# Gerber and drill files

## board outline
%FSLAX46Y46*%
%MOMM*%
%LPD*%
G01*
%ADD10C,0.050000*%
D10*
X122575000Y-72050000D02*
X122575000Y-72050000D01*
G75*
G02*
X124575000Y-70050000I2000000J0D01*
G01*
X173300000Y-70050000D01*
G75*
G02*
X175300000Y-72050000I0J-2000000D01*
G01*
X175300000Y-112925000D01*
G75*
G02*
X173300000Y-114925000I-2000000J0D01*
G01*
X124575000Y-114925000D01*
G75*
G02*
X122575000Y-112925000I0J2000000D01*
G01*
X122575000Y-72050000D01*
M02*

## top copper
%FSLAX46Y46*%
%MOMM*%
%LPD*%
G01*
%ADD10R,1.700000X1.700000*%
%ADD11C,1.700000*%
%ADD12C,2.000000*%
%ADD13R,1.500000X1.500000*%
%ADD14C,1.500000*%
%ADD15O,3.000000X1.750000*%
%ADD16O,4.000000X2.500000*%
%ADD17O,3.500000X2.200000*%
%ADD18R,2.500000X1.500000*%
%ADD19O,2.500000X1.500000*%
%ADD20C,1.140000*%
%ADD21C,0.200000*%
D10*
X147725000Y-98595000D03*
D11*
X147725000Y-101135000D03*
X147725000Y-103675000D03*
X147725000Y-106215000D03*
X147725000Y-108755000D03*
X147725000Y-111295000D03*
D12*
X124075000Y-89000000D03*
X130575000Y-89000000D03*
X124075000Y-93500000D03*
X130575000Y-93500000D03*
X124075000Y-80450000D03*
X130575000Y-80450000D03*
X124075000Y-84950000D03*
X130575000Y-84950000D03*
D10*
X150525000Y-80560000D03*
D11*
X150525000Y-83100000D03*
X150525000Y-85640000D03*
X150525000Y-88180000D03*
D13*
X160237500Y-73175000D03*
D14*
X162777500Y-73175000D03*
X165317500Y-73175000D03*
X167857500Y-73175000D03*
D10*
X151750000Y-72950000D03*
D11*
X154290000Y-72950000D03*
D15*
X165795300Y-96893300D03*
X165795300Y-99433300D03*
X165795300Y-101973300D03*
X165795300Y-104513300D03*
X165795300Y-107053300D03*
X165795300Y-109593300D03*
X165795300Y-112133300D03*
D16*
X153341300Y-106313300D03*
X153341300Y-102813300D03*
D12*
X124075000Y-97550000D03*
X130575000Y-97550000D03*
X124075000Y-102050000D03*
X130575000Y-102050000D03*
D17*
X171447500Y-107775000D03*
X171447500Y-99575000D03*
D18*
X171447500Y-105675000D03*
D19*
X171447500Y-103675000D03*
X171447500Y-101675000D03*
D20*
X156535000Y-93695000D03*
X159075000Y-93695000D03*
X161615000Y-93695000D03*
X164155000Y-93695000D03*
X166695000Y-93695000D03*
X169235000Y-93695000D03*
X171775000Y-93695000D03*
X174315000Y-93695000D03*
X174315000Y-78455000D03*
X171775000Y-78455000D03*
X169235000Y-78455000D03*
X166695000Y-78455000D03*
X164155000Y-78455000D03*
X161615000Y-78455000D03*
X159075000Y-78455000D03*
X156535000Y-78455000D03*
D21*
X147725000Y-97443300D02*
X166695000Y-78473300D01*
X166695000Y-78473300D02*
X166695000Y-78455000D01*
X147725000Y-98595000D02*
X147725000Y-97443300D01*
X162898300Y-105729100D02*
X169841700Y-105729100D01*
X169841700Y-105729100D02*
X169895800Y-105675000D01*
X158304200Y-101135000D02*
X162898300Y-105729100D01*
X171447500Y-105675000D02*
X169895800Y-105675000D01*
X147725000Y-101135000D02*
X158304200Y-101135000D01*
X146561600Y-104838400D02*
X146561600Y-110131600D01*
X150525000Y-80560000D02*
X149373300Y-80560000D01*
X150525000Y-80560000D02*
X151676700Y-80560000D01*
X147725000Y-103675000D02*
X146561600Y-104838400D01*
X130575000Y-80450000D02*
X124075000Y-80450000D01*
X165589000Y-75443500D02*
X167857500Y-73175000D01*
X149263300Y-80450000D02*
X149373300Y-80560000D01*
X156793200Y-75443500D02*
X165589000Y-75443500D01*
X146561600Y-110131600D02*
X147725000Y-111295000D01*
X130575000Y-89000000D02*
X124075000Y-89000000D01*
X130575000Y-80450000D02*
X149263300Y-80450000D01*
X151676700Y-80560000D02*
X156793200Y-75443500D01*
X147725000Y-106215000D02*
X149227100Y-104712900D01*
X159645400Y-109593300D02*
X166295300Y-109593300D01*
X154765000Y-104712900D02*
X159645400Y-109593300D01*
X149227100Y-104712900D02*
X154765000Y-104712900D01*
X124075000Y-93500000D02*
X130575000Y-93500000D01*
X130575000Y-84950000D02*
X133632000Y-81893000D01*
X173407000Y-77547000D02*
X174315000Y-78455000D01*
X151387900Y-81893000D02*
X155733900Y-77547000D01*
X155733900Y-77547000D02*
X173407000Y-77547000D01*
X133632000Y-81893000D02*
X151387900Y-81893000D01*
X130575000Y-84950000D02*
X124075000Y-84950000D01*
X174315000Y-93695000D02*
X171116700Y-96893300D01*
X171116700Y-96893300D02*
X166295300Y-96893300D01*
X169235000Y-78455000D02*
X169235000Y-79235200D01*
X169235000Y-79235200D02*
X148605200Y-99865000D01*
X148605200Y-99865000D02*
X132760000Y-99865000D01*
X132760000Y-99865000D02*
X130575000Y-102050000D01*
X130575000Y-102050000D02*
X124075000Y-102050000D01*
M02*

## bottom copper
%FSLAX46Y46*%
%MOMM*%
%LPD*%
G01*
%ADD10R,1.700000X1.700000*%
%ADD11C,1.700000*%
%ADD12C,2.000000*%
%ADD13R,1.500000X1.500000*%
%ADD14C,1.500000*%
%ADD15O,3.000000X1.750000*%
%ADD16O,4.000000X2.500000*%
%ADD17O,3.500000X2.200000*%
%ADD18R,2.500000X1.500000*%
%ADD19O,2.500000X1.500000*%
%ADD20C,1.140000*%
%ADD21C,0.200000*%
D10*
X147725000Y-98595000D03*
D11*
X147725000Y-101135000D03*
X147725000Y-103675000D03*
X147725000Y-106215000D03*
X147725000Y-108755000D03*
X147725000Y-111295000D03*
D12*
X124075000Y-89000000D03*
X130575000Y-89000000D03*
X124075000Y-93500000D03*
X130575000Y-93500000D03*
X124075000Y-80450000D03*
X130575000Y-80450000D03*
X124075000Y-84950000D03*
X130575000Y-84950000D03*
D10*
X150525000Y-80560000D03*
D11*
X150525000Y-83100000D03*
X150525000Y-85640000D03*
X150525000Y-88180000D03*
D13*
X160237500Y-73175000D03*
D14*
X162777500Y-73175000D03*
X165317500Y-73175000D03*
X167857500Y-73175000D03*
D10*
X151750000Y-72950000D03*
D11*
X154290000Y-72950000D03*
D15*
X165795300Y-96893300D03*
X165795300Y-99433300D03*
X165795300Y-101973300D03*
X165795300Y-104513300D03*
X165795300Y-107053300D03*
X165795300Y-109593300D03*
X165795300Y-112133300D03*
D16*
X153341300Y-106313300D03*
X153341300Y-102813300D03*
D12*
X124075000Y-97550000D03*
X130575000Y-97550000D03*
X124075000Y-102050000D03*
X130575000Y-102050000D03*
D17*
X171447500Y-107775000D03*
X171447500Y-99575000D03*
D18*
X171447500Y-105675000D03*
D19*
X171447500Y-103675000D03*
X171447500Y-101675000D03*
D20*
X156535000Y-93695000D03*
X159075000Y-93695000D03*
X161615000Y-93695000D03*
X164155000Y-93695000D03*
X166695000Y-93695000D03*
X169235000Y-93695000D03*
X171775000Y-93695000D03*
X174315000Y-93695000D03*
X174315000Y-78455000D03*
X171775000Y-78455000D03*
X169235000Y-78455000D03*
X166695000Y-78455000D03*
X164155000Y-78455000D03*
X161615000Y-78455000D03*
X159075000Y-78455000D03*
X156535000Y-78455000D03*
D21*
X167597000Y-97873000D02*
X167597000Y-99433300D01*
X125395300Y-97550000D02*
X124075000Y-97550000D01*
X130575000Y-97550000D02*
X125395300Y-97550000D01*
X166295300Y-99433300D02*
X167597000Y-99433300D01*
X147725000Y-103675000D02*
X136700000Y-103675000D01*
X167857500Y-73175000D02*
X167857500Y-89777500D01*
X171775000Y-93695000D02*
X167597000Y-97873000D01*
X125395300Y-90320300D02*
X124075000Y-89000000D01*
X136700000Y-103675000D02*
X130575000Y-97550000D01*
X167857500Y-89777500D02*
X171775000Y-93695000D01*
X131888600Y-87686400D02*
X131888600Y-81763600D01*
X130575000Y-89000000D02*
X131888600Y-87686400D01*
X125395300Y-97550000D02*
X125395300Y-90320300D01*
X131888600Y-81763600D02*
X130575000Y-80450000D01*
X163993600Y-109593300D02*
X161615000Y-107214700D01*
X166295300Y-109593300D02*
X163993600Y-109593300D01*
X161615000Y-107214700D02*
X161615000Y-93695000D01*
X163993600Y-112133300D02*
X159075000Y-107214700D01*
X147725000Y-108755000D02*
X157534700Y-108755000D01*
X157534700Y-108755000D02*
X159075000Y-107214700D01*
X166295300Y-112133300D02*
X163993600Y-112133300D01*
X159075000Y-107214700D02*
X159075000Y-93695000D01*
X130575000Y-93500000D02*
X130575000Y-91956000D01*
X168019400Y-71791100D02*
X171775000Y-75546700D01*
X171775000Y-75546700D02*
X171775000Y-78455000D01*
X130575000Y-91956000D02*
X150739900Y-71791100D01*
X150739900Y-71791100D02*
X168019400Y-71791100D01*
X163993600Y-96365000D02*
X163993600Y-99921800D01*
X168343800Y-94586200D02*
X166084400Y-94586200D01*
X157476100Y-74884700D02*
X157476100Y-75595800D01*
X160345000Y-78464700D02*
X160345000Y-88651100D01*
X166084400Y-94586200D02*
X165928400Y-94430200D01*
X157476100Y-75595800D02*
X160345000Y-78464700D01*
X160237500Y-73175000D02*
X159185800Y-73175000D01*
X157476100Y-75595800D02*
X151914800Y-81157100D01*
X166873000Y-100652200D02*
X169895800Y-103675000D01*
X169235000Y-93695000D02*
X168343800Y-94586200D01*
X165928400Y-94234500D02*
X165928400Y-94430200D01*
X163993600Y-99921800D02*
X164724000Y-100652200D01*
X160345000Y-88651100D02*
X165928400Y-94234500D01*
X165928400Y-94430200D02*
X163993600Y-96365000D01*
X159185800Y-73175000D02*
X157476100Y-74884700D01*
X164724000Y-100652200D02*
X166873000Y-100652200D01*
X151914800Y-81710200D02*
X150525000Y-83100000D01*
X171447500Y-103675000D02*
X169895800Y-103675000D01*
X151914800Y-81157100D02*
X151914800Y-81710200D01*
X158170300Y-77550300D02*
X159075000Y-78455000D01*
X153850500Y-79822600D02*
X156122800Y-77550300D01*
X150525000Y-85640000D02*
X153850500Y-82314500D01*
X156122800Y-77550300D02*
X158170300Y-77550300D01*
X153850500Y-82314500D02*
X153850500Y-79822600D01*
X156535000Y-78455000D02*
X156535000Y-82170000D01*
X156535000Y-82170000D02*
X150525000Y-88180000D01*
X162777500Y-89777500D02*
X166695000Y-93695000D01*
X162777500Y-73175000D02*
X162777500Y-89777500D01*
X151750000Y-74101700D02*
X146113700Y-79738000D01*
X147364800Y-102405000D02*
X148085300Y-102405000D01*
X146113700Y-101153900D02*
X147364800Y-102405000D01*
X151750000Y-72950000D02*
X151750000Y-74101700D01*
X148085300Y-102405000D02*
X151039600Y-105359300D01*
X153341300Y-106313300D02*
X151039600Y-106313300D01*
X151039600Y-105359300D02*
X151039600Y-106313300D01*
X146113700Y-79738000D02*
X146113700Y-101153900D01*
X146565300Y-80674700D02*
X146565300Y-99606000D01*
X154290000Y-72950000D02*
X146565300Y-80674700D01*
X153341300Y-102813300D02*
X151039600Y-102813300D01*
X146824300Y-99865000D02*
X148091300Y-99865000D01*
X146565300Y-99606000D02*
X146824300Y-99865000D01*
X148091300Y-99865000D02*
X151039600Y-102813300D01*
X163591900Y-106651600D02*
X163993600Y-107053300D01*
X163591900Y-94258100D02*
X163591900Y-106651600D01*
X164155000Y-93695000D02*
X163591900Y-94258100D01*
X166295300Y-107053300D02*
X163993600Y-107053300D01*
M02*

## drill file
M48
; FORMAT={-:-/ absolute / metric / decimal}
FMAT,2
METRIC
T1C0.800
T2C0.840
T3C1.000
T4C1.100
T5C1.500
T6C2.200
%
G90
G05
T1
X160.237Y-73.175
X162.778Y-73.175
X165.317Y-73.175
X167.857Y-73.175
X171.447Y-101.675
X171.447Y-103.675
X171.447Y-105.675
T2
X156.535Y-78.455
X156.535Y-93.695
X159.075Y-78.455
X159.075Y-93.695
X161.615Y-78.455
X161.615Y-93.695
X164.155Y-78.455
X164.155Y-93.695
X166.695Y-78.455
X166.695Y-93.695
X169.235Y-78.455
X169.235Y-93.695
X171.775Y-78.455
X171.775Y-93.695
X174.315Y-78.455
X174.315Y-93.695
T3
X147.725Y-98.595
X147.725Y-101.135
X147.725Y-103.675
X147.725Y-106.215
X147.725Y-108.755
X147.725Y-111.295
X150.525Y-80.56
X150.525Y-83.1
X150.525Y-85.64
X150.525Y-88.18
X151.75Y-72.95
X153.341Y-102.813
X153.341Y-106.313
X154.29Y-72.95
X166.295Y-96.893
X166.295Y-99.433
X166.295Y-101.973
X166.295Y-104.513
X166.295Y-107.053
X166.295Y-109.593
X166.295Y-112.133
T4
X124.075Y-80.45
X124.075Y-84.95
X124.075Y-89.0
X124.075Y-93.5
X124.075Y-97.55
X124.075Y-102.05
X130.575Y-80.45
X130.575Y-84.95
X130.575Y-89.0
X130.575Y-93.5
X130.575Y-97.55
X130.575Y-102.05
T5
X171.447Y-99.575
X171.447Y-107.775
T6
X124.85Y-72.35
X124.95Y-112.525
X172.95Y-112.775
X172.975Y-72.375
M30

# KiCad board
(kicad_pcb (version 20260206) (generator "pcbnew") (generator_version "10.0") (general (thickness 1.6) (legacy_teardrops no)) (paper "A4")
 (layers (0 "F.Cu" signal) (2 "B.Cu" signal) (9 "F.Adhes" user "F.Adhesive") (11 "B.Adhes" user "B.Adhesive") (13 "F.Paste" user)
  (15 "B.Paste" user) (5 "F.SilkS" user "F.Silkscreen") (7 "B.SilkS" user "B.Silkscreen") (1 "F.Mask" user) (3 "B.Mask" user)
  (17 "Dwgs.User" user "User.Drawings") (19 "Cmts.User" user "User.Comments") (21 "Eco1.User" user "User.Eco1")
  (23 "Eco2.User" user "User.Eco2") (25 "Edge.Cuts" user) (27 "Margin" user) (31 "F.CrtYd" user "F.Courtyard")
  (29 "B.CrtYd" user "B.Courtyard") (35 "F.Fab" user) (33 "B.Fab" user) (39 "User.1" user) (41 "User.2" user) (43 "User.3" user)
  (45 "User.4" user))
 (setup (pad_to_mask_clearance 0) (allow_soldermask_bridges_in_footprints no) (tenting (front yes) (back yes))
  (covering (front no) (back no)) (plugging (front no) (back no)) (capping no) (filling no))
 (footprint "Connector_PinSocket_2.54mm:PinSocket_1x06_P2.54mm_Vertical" (layer "F.Cu") (at 147.725 98.595)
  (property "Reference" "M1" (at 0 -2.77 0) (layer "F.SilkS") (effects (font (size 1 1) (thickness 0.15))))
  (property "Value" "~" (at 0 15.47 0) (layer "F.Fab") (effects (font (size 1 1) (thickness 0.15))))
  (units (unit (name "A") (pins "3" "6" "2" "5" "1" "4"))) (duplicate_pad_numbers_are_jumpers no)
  (pad "1" thru_hole rect (at 0 0) (size 1.7 1.7) (drill 1) (layers "*.Cu" "*.Mask") (remove_unused_layers no) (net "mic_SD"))
  (pad "2" thru_hole circle (at 0 2.54) (size 1.7 1.7) (drill 1) (layers "*.Cu" "*.Mask") (remove_unused_layers no) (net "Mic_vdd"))
  (pad "3" thru_hole circle (at 0 5.08) (size 1.7 1.7) (drill 1) (layers "*.Cu" "*.Mask") (remove_unused_layers no) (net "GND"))
  (pad "4" thru_hole circle (at 0 7.62) (size 1.7 1.7) (drill 1) (layers "*.Cu" "*.Mask") (remove_unused_layers no) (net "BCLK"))
  (pad "5" thru_hole circle (at 0 10.16) (size 1.7 1.7) (drill 1) (layers "*.Cu" "*.Mask") (remove_unused_layers no) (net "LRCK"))
  (pad "6" thru_hole circle (at 0 12.7) (size 1.7 1.7) (drill 1) (layers "*.Cu" "*.Mask") (remove_unused_layers no) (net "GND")))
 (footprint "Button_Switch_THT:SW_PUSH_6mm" (layer "F.Cu") (at 124.075 89)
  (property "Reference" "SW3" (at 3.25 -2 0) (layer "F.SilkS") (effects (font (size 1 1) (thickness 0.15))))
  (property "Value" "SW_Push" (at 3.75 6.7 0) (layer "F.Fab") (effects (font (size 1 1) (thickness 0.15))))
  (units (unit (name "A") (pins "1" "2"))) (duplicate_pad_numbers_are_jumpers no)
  (pad "1" thru_hole circle (at 0 0 90) (size 2 2) (drill 1.1) (layers "*.Cu" "*.Mask") (remove_unused_layers no) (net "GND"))
  (pad "1" thru_hole circle (at 6.5 0 90) (size 2 2) (drill 1.1) (layers "*.Cu" "*.Mask") (remove_unused_layers no) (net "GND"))
  (pad "2" thru_hole circle (at 0 4.5 90) (size 2 2) (drill 1.1) (layers "*.Cu" "*.Mask") (remove_unused_layers no) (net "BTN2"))
  (pad "2" thru_hole circle (at 6.5 4.5 90) (size 2 2) (drill 1.1) (layers "*.Cu" "*.Mask") (remove_unused_layers no) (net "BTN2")))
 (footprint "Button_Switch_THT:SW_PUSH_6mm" (layer "F.Cu") (at 124.075 80.45)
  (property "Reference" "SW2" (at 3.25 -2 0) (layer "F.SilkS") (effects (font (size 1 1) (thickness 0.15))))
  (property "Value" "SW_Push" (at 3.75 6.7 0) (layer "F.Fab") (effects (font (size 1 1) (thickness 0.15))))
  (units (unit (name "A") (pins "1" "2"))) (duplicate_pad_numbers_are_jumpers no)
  (pad "1" thru_hole circle (at 0 0 90) (size 2 2) (drill 1.1) (layers "*.Cu" "*.Mask") (remove_unused_layers no) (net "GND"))
  (pad "1" thru_hole circle (at 6.5 0 90) (size 2 2) (drill 1.1) (layers "*.Cu" "*.Mask") (remove_unused_layers no) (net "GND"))
  (pad "2" thru_hole circle (at 0 4.5 90) (size 2 2) (drill 1.1) (layers "*.Cu" "*.Mask") (remove_unused_layers no) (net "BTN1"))
  (pad "2" thru_hole circle (at 6.5 4.5 90) (size 2 2) (drill 1.1) (layers "*.Cu" "*.Mask") (remove_unused_layers no) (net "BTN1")))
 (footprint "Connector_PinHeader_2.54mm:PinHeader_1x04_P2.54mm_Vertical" (layer "F.Cu") (at 150.525 80.56)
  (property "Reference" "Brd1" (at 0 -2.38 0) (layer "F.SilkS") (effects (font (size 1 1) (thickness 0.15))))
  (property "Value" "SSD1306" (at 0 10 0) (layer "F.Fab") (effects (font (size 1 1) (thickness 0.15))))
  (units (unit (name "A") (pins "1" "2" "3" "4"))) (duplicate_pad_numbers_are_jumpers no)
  (pad "1" thru_hole rect (at 0 0) (size 1.7 1.7) (drill 1) (layers "*.Cu" "*.Mask") (remove_unused_layers no) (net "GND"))
  (pad "2" thru_hole circle (at 0 2.54) (size 1.7 1.7) (drill 1) (layers "*.Cu" "*.Mask") (remove_unused_layers no) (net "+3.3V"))
  (pad "3" thru_hole circle (at 0 5.08) (size 1.7 1.7) (drill 1) (layers "*.Cu" "*.Mask") (remove_unused_layers no) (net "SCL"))
  (pad "4" thru_hole circle (at 0 7.62) (size 1.7 1.7) (drill 1) (layers "*.Cu" "*.Mask") (remove_unused_layers no) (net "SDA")))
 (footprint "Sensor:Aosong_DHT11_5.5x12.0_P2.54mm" (layer "F.Cu") (at 160.2375 73.175 90)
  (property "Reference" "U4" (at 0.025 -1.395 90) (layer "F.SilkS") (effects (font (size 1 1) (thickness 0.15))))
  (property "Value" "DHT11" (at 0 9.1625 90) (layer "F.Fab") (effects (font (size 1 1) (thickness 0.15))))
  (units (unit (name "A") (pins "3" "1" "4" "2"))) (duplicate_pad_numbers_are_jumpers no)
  (pad "1" thru_hole rect (at 0 0 90) (size 1.5 1.5) (drill 0.8) (layers "*.Cu" "*.Mask") (remove_unused_layers no) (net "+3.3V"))
  (pad "2" thru_hole circle (at 0 2.54 90) (size 1.5 1.5) (drill 0.8) (layers "*.Cu" "*.Mask") (remove_unused_layers no) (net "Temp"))
  (pad "3" thru_hole circle (at 0 5.08 90) (size 1.5 1.5) (drill 0.8) (layers "*.Cu" "*.Mask") (remove_unused_layers no)
   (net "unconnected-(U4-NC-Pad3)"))
  (pad "4" thru_hole circle (at 0 7.62 90) (size 1.5 1.5) (drill 0.8) (layers "*.Cu" "*.Mask") (remove_unused_layers no) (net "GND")))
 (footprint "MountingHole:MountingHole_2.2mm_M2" (layer "F.Cu") (at 172.975 72.375)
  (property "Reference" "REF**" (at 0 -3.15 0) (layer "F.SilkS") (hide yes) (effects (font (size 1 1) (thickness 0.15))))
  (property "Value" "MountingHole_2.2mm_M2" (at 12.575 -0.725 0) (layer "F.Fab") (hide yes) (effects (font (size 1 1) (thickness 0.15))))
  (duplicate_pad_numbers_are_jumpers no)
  (pad "" np_thru_hole circle (at 0 0) (size 2.2 2.2) (drill 2.2) (layers "*.Cu" "*.Mask")))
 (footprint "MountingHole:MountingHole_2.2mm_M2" (layer "F.Cu") (at 124.95 112.525)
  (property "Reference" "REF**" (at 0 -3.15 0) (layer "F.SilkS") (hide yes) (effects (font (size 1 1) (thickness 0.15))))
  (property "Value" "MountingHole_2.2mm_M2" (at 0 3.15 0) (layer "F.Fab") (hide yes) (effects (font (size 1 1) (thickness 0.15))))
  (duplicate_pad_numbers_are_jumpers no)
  (pad "" np_thru_hole circle (at 0 0) (size 2.2 2.2) (drill 2.2) (layers "*.Cu" "*.Mask")))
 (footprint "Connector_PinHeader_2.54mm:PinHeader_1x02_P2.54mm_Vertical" (layer "F.Cu") (at 151.75 72.95 90)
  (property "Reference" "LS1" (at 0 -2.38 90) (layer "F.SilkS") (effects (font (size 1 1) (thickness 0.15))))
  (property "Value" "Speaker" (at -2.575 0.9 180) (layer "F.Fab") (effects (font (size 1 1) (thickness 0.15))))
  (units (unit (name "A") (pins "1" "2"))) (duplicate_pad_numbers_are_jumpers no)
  (pad "1" thru_hole rect (at 0 0 90) (size 1.7 1.7) (drill 1) (layers "*.Cu" "*.Mask") (remove_unused_layers no) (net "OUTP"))
  (pad "2" thru_hole circle (at 0 2.54 90) (size 1.7 1.7) (drill 1) (layers "*.Cu" "*.Mask") (remove_unused_layers no) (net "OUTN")))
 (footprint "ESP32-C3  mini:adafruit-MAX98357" (layer "F.Cu") (at 159.3883 104.3933 90)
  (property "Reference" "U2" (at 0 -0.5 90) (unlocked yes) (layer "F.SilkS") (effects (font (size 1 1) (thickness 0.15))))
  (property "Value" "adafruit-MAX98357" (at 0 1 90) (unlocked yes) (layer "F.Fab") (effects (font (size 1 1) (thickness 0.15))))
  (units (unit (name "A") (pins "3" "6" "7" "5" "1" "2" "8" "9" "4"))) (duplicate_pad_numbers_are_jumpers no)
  (pad "1" thru_hole oval (at 7.5 6.907) (size 3 1.75) (drill 1 (offset -0.5 0)) (layers "*.Cu" "*.Mask") (remove_unused_layers no)
   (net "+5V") (solder_mask_margin 0.0508))
  (pad "2" thru_hole oval (at 4.96 6.907) (size 3 1.75) (drill 1 (offset -0.5 0)) (layers "*.Cu" "*.Mask") (remove_unused_layers no)
   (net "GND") (solder_mask_margin 0.0508))
  (pad "3" thru_hole oval (at 2.42 6.907) (size 3 1.75) (drill 1 (offset -0.5 0)) (layers "*.Cu" "*.Mask") (remove_unused_layers no)
   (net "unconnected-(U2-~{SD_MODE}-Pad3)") (solder_mask_margin 0.0508))
  (pad "4" thru_hole oval (at -0.12 6.907) (size 3 1.75) (drill 1 (offset -0.5 0)) (layers "*.Cu" "*.Mask") (remove_unused_layers no)
   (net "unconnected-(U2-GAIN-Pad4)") (solder_mask_margin 0.0508))
  (pad "5" thru_hole oval (at -2.66 6.907) (size 3 1.75) (drill 1 (offset -0.5 0)) (layers "*.Cu" "*.Mask") (remove_unused_layers no)
   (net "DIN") (solder_mask_margin 0.0508))
  (pad "6" thru_hole oval (at -5.2 6.907) (size 3 1.75) (drill 1 (offset -0.5 0)) (layers "*.Cu" "*.Mask") (remove_unused_layers no)
   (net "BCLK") (solder_mask_margin 0.0508))
  (pad "7" thru_hole oval (at -7.74 6.907) (size 3 1.75) (drill 1 (offset -0.5 0)) (layers "*.Cu" "*.Mask") (remove_unused_layers no)
   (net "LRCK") (solder_mask_margin 0.0508))
  (pad "8" thru_hole oval (at -1.92 -6.047 270) (size 2.5 4) (drill 1) (layers "*.Cu" "*.Mask") (remove_unused_layers no) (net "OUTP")
   (solder_mask_margin 0.0508))
  (pad "9" thru_hole oval (at 1.58 -6.047 270) (size 2.5 4) (drill 1) (layers "*.Cu" "*.Mask") (remove_unused_layers no) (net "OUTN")
   (solder_mask_margin 0.0508)))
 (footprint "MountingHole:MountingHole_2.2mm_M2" (layer "F.Cu") (at 172.95 112.775)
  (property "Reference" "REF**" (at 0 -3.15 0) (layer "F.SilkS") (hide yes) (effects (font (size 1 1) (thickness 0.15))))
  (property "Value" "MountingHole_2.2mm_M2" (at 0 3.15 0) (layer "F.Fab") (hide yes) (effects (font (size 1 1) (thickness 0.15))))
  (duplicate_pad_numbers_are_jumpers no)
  (pad "" np_thru_hole circle (at 0 0) (size 2.2 2.2) (drill 2.2) (layers "*.Cu" "*.Mask")))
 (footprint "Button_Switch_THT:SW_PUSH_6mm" (layer "F.Cu") (at 124.075 97.55)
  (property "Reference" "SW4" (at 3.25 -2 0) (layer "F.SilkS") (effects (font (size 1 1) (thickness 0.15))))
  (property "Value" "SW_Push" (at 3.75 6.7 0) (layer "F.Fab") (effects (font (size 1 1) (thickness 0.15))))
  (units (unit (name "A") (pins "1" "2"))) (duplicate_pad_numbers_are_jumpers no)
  (pad "1" thru_hole circle (at 0 0 90) (size 2 2) (drill 1.1) (layers "*.Cu" "*.Mask") (remove_unused_layers no) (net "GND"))
  (pad "1" thru_hole circle (at 6.5 0 90) (size 2 2) (drill 1.1) (layers "*.Cu" "*.Mask") (remove_unused_layers no) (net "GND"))
  (pad "2" thru_hole circle (at 0 4.5 90) (size 2 2) (drill 1.1) (layers "*.Cu" "*.Mask") (remove_unused_layers no) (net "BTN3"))
  (pad "2" thru_hole circle (at 6.5 4.5 90) (size 2 2) (drill 1.1) (layers "*.Cu" "*.Mask") (remove_unused_layers no) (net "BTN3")))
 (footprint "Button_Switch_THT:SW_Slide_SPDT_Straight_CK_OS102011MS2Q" (layer "F.Cu") (at 171.4475 105.675 90)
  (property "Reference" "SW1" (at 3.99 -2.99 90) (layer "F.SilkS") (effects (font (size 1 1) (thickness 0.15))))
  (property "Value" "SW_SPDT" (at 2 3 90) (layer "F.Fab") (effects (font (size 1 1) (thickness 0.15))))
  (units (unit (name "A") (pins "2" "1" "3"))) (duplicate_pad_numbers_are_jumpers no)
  (pad "" thru_hole oval (at -2.1 0 90) (size 2.2 3.5) (drill 1.5) (layers "*.Cu" "*.Mask") (remove_unused_layers no))
  (pad "" thru_hole oval (at 6.1 0 90) (size 2.2 3.5) (drill 1.5) (layers "*.Cu" "*.Mask") (remove_unused_layers no))
  (pad "1" thru_hole rect (at 0 0 90) (size 1.5 2.5) (drill 0.8) (layers "*.Cu" "*.Mask") (remove_unused_layers no) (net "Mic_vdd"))
  (pad "2" thru_hole oval (at 2 0 90) (size 1.5 2.5) (drill 0.8) (layers "*.Cu" "*.Mask") (remove_unused_layers no) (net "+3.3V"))
  (pad "3" thru_hole oval (at 4 0 90) (size 1.5 2.5) (drill 0.8) (layers "*.Cu" "*.Mask") (remove_unused_layers no)
   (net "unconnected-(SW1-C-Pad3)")))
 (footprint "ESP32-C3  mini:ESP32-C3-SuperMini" (layer "F.Cu") (at 165.425 86.075 -90)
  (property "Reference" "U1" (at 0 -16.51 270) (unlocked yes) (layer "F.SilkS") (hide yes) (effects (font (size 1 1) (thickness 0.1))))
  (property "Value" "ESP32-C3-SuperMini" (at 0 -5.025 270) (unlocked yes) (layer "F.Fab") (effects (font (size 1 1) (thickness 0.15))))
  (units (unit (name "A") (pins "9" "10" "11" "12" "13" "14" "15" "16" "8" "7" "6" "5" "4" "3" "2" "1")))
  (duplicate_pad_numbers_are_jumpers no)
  (pad "1" thru_hole circle (at 7.62 8.89 270) (size 1.14 1.14) (drill 0.84) (layers "*.Cu" "*.Mask") (remove_unused_layers no)
   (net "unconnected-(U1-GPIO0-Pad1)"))
  (pad "2" thru_hole circle (at 7.62 6.35 270) (size 1.14 1.14) (drill 0.84) (layers "*.Cu" "*.Mask") (remove_unused_layers no) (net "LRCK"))
  (pad "3" thru_hole circle (at 7.62 3.81 270) (size 1.14 1.14) (drill 0.84) (layers "*.Cu" "*.Mask") (remove_unused_layers no) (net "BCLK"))
  (pad "4" thru_hole circle (at 7.62 1.27 270) (size 1.14 1.14) (drill 0.84) (layers "*.Cu" "*.Mask") (remove_unused_layers no) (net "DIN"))
  (pad "5" thru_hole circle (at 7.62 -1.27 270) (size 1.14 1.14) (drill 0.84) (layers "*.Cu" "*.Mask") (remove_unused_layers no)
   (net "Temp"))
  (pad "6" thru_hole circle (at 7.62 -3.81 270) (size 1.14 1.14) (drill 0.84) (layers "*.Cu" "*.Mask") (remove_unused_layers no)
   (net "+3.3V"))
  (pad "7" thru_hole circle (at 7.62 -6.35 270) (size 1.14 1.14) (drill 0.84) (layers "*.Cu" "*.Mask") (remove_unused_layers no) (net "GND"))
  (pad "8" thru_hole circle (at 7.62 -8.89 270) (size 1.14 1.14) (drill 0.84) (layers "*.Cu" "*.Mask") (remove_unused_layers no) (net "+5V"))
  (pad "9" thru_hole circle (at -7.62 -8.89 270) (size 1.14 1.14) (drill 0.84) (layers "*.Cu" "*.Mask") (remove_unused_layers no)
   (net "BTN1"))
  (pad "10" thru_hole circle (at -7.62 -6.35 270) (size 1.14 1.14) (drill 0.84) (layers "*.Cu" "*.Mask") (remove_unused_layers no)
   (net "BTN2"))
  (pad "11" thru_hole circle (at -7.62 -3.81 270) (size 1.14 1.14) (drill 0.84) (layers "*.Cu" "*.Mask") (remove_unused_layers no)
   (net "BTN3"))
  (pad "12" thru_hole circle (at -7.62 -1.27 270) (size 1.14 1.14) (drill 0.84) (layers "*.Cu" "*.Mask") (remove_unused_layers no)
   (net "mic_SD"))
  (pad "13" thru_hole circle (at -7.62 1.27 270) (size 1.14 1.14) (drill 0.84) (layers "*.Cu" "*.Mask") (remove_unused_layers no)
   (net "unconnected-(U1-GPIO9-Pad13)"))
  (pad "14" thru_hole circle (at -7.62 3.81 270) (size 1.14 1.14) (drill 0.84) (layers "*.Cu" "*.Mask") (remove_unused_layers no)
   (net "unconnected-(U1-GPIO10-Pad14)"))
  (pad "15" thru_hole circle (at -7.62 6.35 270) (size 1.14 1.14) (drill 0.84) (layers "*.Cu" "*.Mask") (remove_unused_layers no)
   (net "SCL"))
  (pad "16" thru_hole circle (at -7.62 8.89 270) (size 1.14 1.14) (drill 0.84) (layers "*.Cu" "*.Mask") (remove_unused_layers no)
   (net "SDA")))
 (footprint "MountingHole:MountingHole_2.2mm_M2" (layer "F.Cu") (at 124.85 72.35)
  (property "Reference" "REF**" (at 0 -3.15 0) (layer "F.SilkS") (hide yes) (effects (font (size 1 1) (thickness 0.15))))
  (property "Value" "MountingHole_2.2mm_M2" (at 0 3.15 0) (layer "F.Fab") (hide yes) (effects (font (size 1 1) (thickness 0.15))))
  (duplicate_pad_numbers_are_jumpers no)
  (pad "" np_thru_hole circle (at 0 0) (size 2.2 2.2) (drill 2.2) (layers "*.Cu" "*.Mask")))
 (gr_rect (start 122.575 70.05) (end 175.3 114.925) (radius 2) (stroke (width 0.05) (type solid)) (fill no) (layer "Edge.Cuts"))
 (segment (start 147.725 97.4433) (end 166.695 78.4733) (width 0.2) (layer "F.Cu") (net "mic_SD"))
 (segment (start 166.695 78.4733) (end 166.695 78.455) (width 0.2) (layer "F.Cu") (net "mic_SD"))
 (segment (start 147.725 98.595) (end 147.725 97.4433) (width 0.2) (layer "F.Cu") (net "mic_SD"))
 (segment (start 162.8983 105.7291) (end 169.8417 105.7291) (width 0.2) (layer "F.Cu") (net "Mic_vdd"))
 (segment (start 169.8417 105.7291) (end 169.8958 105.675) (width 0.2) (layer "F.Cu") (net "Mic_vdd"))
 (segment (start 158.3042 101.135) (end 162.8983 105.7291) (width 0.2) (layer "F.Cu") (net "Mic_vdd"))
 (segment (start 171.4475 105.675) (end 169.8958 105.675) (width 0.2) (layer "F.Cu") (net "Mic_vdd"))
 (segment (start 147.725 101.135) (end 158.3042 101.135) (width 0.2) (layer "F.Cu") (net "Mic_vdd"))
 (segment (start 146.5616 104.8384) (end 146.5616 110.1316) (width 0.2) (layer "F.Cu") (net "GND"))
 (segment (start 150.525 80.56) (end 149.3733 80.56) (width 0.2) (layer "F.Cu") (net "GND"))
 (segment (start 150.525 80.56) (end 151.6767 80.56) (width 0.2) (layer "F.Cu") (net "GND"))
 (segment (start 147.725 103.675) (end 146.5616 104.8384) (width 0.2) (layer "F.Cu") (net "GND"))
 (segment (start 130.575 80.45) (end 124.075 80.45) (width 0.2) (layer "F.Cu") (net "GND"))
 (segment (start 165.589 75.4435) (end 167.8575 73.175) (width 0.2) (layer "F.Cu") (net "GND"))
 (segment (start 149.2633 80.45) (end 149.3733 80.56) (width 0.2) (layer "F.Cu") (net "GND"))
 (segment (start 156.7932 75.4435) (end 165.589 75.4435) (width 0.2) (layer "F.Cu") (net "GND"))
 (segment (start 146.5616 110.1316) (end 147.725 111.295) (width 0.2) (layer "F.Cu") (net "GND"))
 (segment (start 130.575 89) (end 124.075 89) (width 0.2) (layer "F.Cu") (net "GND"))
 (segment (start 130.575 80.45) (end 149.2633 80.45) (width 0.2) (layer "F.Cu") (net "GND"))
 (segment (start 151.6767 80.56) (end 156.7932 75.4435) (width 0.2) (layer "F.Cu") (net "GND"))
 (segment (start 167.597 97.873) (end 167.597 99.4333) (width 0.2) (layer "B.Cu") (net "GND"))
 (segment (start 125.3953 97.55) (end 124.075 97.55) (width 0.2) (layer "B.Cu") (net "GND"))
 (segment (start 130.575 97.55) (end 125.3953 97.55) (width 0.2) (layer "B.Cu") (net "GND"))
 (segment (start 166.2953 99.4333) (end 167.597 99.4333) (width 0.2) (layer "B.Cu") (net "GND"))
 (segment (start 147.725 103.675) (end 136.7 103.675) (width 0.2) (layer "B.Cu") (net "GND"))
 (segment (start 167.8575 73.175) (end 167.8575 89.7775) (width 0.2) (layer "B.Cu") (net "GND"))
 (segment (start 171.775 93.695) (end 167.597 97.873) (width 0.2) (layer "B.Cu") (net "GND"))
 (segment (start 125.3953 90.3203) (end 124.075 89) (width 0.2) (layer "B.Cu") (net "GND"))
 (segment (start 136.7 103.675) (end 130.575 97.55) (width 0.2) (layer "B.Cu") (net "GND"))
 (segment (start 167.8575 89.7775) (end 171.775 93.695) (width 0.2) (layer "B.Cu") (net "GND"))
 (segment (start 131.8886 87.6864) (end 131.8886 81.7636) (width 0.2) (layer "B.Cu") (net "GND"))
 (segment (start 130.575 89) (end 131.8886 87.6864) (width 0.2) (layer "B.Cu") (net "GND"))
 (segment (start 125.3953 97.55) (end 125.3953 90.3203) (width 0.2) (layer "B.Cu") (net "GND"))
 (segment (start 131.8886 81.7636) (end 130.575 80.45) (width 0.2) (layer "B.Cu") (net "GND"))
 (segment (start 147.725 106.215) (end 149.2271 104.7129) (width 0.2) (layer "F.Cu") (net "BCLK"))
 (segment (start 159.6454 109.5933) (end 166.2953 109.5933) (width 0.2) (layer "F.Cu") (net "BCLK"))
 (segment (start 154.765 104.7129) (end 159.6454 109.5933) (width 0.2) (layer "F.Cu") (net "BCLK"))
 (segment (start 149.2271 104.7129) (end 154.765 104.7129) (width 0.2) (layer "F.Cu") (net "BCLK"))
 (segment (start 163.9936 109.5933) (end 161.615 107.2147) (width 0.2) (layer "B.Cu") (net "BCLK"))
 (segment (start 166.2953 109.5933) (end 163.9936 109.5933) (width 0.2) (layer "B.Cu") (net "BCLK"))
 (segment (start 161.615 107.2147) (end 161.615 93.695) (width 0.2) (layer "B.Cu") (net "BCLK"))
 (segment (start 163.9936 112.1333) (end 159.075 107.2147) (width 0.2) (layer "B.Cu") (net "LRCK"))
 (segment (start 147.725 108.755) (end 157.5347 108.755) (width 0.2) (layer "B.Cu") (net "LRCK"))
 (segment (start 157.5347 108.755) (end 159.075 107.2147) (width 0.2) (layer "B.Cu") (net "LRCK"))
 (segment (start 166.2953 112.1333) (end 163.9936 112.1333) (width 0.2) (layer "B.Cu") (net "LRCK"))
 (segment (start 159.075 107.2147) (end 159.075 93.695) (width 0.2) (layer "B.Cu") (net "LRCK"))
 (segment (start 124.075 93.5) (end 130.575 93.5) (width 0.2) (layer "F.Cu") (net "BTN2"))
 (segment (start 130.575 93.5) (end 130.575 91.956) (width 0.2) (layer "B.Cu") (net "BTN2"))
 (segment (start 168.0194 71.7911) (end 171.775 75.5467) (width 0.2) (layer "B.Cu") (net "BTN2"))
 (segment (start 171.775 75.5467) (end 171.775 78.455) (width 0.2) (layer "B.Cu") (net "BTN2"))
 (segment (start 130.575 91.956) (end 150.7399 71.7911) (width 0.2) (layer "B.Cu") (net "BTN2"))
 (segment (start 150.7399 71.7911) (end 168.0194 71.7911) (width 0.2) (layer "B.Cu") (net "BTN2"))
 (segment (start 130.575 84.95) (end 133.632 81.893) (width 0.2) (layer "F.Cu") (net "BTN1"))
 (segment (start 173.407 77.547) (end 174.315 78.455) (width 0.2) (layer "F.Cu") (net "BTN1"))
 (segment (start 151.3879 81.893) (end 155.7339 77.547) (width 0.2) (layer "F.Cu") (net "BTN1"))
 (segment (start 155.7339 77.547) (end 173.407 77.547) (width 0.2) (layer "F.Cu") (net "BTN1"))
 (segment (start 133.632 81.893) (end 151.3879 81.893) (width 0.2) (layer "F.Cu") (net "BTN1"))
 (segment (start 130.575 84.95) (end 124.075 84.95) (width 0.2) (layer "F.Cu") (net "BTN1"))
 (segment (start 163.9936 96.365) (end 163.9936 99.9218) (width 0.2) (layer "B.Cu") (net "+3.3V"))
 (segment (start 168.3438 94.5862) (end 166.0844 94.5862) (width 0.2) (layer "B.Cu") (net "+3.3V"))
 (segment (start 157.4761 74.8847) (end 157.4761 75.5958) (width 0.2) (layer "B.Cu") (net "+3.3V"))
 (segment (start 160.345 78.4647) (end 160.345 88.6511) (width 0.2) (layer "B.Cu") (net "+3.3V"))
 (segment (start 166.0844 94.5862) (end 165.9284 94.4302) (width 0.2) (layer "B.Cu") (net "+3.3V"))
 (segment (start 157.4761 75.5958) (end 160.345 78.4647) (width 0.2) (layer "B.Cu") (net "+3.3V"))
 (segment (start 160.2375 73.175) (end 159.1858 73.175) (width 0.2) (layer "B.Cu") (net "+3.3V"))
 (segment (start 157.4761 75.5958) (end 151.9148 81.1571) (width 0.2) (layer "B.Cu") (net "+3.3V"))
 (segment (start 166.873 100.6522) (end 169.8958 103.675) (width 0.2) (layer "B.Cu") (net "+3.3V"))
 (segment (start 169.235 93.695) (end 168.3438 94.5862) (width 0.2) (layer "B.Cu") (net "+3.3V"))
 (segment (start 165.9284 94.2345) (end 165.9284 94.4302) (width 0.2) (layer "B.Cu") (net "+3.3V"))
 (segment (start 163.9936 99.9218) (end 164.724 100.6522) (width 0.2) (layer "B.Cu") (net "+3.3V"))
 (segment (start 160.345 88.6511) (end 165.9284 94.2345) (width 0.2) (layer "B.Cu") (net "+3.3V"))
 (segment (start 165.9284 94.4302) (end 163.9936 96.365) (width 0.2) (layer "B.Cu") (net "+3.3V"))
 (segment (start 159.1858 73.175) (end 157.4761 74.8847) (width 0.2) (layer "B.Cu") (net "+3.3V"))
 (segment (start 164.724 100.6522) (end 166.873 100.6522) (width 0.2) (layer "B.Cu") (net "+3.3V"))
 (segment (start 151.9148 81.7102) (end 150.525 83.1) (width 0.2) (layer "B.Cu") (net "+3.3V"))
 (segment (start 171.4475 103.675) (end 169.8958 103.675) (width 0.2) (layer "B.Cu") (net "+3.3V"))
 (segment (start 151.9148 81.1571) (end 151.9148 81.7102) (width 0.2) (layer "B.Cu") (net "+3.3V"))
 (segment (start 158.1703 77.5503) (end 159.075 78.455) (width 0.2) (layer "B.Cu") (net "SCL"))
 (segment (start 153.8505 79.8226) (end 156.1228 77.5503) (width 0.2) (layer "B.Cu") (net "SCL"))
 (segment (start 150.525 85.64) (end 153.8505 82.3145) (width 0.2) (layer "B.Cu") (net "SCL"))
 (segment (start 156.1228 77.5503) (end 158.1703 77.5503) (width 0.2) (layer "B.Cu") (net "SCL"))
 (segment (start 153.8505 82.3145) (end 153.8505 79.8226) (width 0.2) (layer "B.Cu") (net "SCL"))
 (segment (start 156.535 78.455) (end 156.535 82.17) (width 0.2) (layer "B.Cu") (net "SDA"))
 (segment (start 156.535 82.17) (end 150.525 88.18) (width 0.2) (layer "B.Cu") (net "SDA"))
 (segment (start 162.7775 89.7775) (end 166.695 93.695) (width 0.2) (layer "B.Cu") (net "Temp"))
 (segment (start 162.7775 73.175) (end 162.7775 89.7775) (width 0.2) (layer "B.Cu") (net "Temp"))
 (segment (start 151.75 74.1017) (end 146.1137 79.738) (width 0.2) (layer "B.Cu") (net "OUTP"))
 (segment (start 147.3648 102.405) (end 148.0853 102.405) (width 0.2) (layer "B.Cu") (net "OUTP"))
 (segment (start 146.1137 101.1539) (end 147.3648 102.405) (width 0.2) (layer "B.Cu") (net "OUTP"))
 (segment (start 151.75 72.95) (end 151.75 74.1017) (width 0.2) (layer "B.Cu") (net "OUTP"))
 (segment (start 148.0853 102.405) (end 151.0396 105.3593) (width 0.2) (layer "B.Cu") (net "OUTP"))
 (segment (start 153.3413 106.3133) (end 151.0396 106.3133) (width 0.2) (layer "B.Cu") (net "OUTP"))
 (segment (start 151.0396 105.3593) (end 151.0396 106.3133) (width 0.2) (layer "B.Cu") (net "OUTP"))
 (segment (start 146.1137 79.738) (end 146.1137 101.1539) (width 0.2) (layer "B.Cu") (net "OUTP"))
 (segment (start 146.5653 80.6747) (end 146.5653 99.606) (width 0.2) (layer "B.Cu") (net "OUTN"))
 (segment (start 154.29 72.95) (end 146.5653 80.6747) (width 0.2) (layer "B.Cu") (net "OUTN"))
 (segment (start 153.3413 102.8133) (end 151.0396 102.8133) (width 0.2) (layer "B.Cu") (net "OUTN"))
 (segment (start 146.8243 99.865) (end 148.0913 99.865) (width 0.2) (layer "B.Cu") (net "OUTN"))
 (segment (start 146.5653 99.606) (end 146.8243 99.865) (width 0.2) (layer "B.Cu") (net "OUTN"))
 (segment (start 148.0913 99.865) (end 151.0396 102.8133) (width 0.2) (layer "B.Cu") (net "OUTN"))
 (segment (start 174.315 93.695) (end 171.1167 96.8933) (width 0.2) (layer "F.Cu") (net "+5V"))
 (segment (start 171.1167 96.8933) (end 166.2953 96.8933) (width 0.2) (layer "F.Cu") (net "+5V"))
 (segment (start 163.5919 106.6516) (end 163.9936 107.0533) (width 0.2) (layer "B.Cu") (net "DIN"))
 (segment (start 163.5919 94.2581) (end 163.5919 106.6516) (width 0.2) (layer "B.Cu") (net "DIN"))
 (segment (start 164.155 93.695) (end 163.5919 94.2581) (width 0.2) (layer "B.Cu") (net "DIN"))
 (segment (start 166.2953 107.0533) (end 163.9936 107.0533) (width 0.2) (layer "B.Cu") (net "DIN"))
 (segment (start 169.235 78.455) (end 169.235 79.2352) (width 0.2) (layer "F.Cu") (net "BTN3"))
 (segment (start 169.235 79.2352) (end 148.6052 99.865) (width 0.2) (layer "F.Cu") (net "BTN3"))
 (segment (start 148.6052 99.865) (end 132.76 99.865) (width 0.2) (layer "F.Cu") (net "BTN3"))
 (segment (start 132.76 99.865) (end 130.575 102.05) (width 0.2) (layer "F.Cu") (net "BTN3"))
 (segment (start 130.575 102.05) (end 124.075 102.05) (width 0.2) (layer "F.Cu") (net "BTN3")))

